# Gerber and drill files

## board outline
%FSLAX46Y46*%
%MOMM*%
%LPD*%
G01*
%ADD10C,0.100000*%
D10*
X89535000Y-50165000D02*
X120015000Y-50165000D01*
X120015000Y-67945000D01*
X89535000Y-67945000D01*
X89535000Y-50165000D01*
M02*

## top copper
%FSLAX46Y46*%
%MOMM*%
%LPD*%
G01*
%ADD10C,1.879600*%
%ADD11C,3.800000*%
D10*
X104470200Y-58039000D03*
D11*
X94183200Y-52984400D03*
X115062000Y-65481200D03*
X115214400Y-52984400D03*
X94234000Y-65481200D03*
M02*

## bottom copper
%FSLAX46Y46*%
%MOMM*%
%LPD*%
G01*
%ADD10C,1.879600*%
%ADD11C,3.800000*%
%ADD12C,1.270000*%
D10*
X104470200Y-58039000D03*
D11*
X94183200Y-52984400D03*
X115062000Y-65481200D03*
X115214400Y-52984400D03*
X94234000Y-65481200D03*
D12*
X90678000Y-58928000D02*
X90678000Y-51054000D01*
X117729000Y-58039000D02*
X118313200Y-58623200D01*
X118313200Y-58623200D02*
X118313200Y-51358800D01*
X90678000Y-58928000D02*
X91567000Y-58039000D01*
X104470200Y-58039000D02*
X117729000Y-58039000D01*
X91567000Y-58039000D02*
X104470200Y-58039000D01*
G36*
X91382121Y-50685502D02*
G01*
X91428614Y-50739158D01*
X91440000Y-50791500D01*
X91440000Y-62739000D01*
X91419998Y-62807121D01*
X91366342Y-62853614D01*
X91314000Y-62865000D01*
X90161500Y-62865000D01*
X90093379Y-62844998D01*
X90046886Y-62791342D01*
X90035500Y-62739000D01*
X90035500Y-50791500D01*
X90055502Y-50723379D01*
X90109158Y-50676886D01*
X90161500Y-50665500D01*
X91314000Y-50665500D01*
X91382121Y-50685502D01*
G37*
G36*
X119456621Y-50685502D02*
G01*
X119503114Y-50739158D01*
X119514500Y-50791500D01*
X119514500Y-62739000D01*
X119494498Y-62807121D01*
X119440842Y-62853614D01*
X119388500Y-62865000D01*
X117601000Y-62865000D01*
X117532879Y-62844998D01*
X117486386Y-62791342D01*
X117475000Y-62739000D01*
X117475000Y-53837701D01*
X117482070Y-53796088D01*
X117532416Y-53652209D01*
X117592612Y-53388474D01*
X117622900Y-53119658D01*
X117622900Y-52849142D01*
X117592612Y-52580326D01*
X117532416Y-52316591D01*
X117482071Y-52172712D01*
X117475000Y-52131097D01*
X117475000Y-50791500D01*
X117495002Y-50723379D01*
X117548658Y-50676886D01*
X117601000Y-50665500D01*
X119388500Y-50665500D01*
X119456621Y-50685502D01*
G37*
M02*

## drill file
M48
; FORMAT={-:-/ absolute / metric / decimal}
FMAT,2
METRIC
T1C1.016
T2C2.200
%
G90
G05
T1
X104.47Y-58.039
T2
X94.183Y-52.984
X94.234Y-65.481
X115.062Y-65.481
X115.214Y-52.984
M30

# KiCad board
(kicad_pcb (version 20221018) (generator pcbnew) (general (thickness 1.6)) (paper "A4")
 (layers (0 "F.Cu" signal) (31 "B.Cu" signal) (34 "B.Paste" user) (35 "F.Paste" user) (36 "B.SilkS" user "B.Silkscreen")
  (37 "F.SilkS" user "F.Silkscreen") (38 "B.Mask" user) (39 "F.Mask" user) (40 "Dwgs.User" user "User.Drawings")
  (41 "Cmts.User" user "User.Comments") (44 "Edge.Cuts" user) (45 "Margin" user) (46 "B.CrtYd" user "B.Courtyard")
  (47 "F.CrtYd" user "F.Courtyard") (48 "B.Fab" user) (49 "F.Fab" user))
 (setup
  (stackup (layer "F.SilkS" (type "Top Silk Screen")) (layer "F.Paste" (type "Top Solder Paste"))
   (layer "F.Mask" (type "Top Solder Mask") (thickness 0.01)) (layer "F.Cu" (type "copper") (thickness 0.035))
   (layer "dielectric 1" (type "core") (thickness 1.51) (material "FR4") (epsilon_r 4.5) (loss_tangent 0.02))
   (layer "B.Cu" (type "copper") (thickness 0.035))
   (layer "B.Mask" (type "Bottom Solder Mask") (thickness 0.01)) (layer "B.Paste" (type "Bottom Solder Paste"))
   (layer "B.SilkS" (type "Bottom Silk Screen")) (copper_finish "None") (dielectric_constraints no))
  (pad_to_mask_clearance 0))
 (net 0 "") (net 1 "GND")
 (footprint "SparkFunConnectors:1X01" (layer "F.Cu") (at 104.4702 58.039)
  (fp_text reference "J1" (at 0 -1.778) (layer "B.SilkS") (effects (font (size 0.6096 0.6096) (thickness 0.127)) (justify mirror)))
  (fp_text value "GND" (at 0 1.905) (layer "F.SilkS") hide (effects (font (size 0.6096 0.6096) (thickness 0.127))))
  (pad "1" thru_hole circle (at 0 0) (size 1.8796 1.8796) (drill 1.016) (layers "*.Cu" "*.Mask") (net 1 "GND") (solder_mask_margin 0.1016)))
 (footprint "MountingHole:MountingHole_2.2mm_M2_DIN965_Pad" (layer "F.Cu") (at 94.1832 52.9844)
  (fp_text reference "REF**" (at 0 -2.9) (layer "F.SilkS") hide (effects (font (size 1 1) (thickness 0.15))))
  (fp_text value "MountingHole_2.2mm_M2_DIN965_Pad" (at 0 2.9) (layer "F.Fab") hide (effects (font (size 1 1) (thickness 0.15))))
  (pad "1" thru_hole circle (at 0 0) (size 3.8 3.8) (drill 2.2) (layers "*.Cu" "*.Mask")))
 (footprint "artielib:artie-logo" (layer "F.Cu") (at 110.363 58.166)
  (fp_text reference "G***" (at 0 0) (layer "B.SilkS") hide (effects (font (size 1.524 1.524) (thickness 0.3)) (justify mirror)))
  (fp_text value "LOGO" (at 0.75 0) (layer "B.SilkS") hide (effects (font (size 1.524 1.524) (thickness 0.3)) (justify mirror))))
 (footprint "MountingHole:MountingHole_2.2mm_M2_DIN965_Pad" (layer "F.Cu") (at 115.062 65.4812)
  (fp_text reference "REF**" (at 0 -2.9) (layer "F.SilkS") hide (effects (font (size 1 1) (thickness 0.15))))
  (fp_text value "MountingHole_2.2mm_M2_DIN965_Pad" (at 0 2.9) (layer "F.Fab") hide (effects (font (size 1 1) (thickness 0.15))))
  (pad "1" thru_hole circle (at 0 0) (size 3.8 3.8) (drill 2.2) (layers "*.Cu" "*.Mask")))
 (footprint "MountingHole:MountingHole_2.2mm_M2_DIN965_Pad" (layer "F.Cu") (at 115.2144 52.9844)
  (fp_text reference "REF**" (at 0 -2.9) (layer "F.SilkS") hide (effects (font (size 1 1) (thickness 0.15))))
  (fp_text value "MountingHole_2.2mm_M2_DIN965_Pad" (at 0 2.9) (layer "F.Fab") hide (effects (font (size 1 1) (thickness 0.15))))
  (pad "1" thru_hole circle (at 0 0) (size 3.8 3.8) (drill 2.2) (layers "*.Cu" "*.Mask")))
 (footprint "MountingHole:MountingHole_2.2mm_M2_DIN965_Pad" (layer "F.Cu") (at 94.234 65.4812)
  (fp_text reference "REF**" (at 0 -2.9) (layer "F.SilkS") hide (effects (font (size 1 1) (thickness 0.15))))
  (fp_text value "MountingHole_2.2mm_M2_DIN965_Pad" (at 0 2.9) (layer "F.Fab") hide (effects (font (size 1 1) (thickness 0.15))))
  (pad "1" thru_hole circle (at 0 0) (size 3.8 3.8) (drill 2.2) (layers "*.Cu" "*.Mask")))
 (gr_rect (start 89.535 50.165) (end 120.015 67.945) (stroke (width 0.1) (type solid)) (fill none) (layer "Edge.Cuts"))
 (segment (start 90.678 58.928) (end 90.678 51.054) (width 1.27) (layer "B.Cu") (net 1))
 (segment (start 117.729 58.039) (end 118.3132 58.6232) (width 1.27) (layer "B.Cu") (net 1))
 (segment (start 118.3132 58.6232) (end 118.3132 51.3588) (width 1.27) (layer "B.Cu") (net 1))
 (segment (start 90.678 58.928) (end 91.567 58.039) (width 1.27) (layer "B.Cu") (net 1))
 (segment (start 104.4702 58.039) (end 117.729 58.039) (width 1.27) (layer "B.Cu") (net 1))
 (segment (start 91.567 58.039) (end 104.4702 58.039) (width 1.27) (layer "B.Cu") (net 1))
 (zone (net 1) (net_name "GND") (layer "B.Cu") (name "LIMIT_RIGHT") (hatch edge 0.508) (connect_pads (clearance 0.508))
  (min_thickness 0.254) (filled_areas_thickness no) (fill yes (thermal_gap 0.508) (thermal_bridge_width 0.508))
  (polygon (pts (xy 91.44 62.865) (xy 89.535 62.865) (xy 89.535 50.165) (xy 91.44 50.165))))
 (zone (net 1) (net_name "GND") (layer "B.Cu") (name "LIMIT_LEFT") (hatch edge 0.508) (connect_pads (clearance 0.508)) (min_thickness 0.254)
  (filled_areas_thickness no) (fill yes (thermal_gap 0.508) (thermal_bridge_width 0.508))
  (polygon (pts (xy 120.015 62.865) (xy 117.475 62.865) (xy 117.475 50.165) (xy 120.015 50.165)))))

